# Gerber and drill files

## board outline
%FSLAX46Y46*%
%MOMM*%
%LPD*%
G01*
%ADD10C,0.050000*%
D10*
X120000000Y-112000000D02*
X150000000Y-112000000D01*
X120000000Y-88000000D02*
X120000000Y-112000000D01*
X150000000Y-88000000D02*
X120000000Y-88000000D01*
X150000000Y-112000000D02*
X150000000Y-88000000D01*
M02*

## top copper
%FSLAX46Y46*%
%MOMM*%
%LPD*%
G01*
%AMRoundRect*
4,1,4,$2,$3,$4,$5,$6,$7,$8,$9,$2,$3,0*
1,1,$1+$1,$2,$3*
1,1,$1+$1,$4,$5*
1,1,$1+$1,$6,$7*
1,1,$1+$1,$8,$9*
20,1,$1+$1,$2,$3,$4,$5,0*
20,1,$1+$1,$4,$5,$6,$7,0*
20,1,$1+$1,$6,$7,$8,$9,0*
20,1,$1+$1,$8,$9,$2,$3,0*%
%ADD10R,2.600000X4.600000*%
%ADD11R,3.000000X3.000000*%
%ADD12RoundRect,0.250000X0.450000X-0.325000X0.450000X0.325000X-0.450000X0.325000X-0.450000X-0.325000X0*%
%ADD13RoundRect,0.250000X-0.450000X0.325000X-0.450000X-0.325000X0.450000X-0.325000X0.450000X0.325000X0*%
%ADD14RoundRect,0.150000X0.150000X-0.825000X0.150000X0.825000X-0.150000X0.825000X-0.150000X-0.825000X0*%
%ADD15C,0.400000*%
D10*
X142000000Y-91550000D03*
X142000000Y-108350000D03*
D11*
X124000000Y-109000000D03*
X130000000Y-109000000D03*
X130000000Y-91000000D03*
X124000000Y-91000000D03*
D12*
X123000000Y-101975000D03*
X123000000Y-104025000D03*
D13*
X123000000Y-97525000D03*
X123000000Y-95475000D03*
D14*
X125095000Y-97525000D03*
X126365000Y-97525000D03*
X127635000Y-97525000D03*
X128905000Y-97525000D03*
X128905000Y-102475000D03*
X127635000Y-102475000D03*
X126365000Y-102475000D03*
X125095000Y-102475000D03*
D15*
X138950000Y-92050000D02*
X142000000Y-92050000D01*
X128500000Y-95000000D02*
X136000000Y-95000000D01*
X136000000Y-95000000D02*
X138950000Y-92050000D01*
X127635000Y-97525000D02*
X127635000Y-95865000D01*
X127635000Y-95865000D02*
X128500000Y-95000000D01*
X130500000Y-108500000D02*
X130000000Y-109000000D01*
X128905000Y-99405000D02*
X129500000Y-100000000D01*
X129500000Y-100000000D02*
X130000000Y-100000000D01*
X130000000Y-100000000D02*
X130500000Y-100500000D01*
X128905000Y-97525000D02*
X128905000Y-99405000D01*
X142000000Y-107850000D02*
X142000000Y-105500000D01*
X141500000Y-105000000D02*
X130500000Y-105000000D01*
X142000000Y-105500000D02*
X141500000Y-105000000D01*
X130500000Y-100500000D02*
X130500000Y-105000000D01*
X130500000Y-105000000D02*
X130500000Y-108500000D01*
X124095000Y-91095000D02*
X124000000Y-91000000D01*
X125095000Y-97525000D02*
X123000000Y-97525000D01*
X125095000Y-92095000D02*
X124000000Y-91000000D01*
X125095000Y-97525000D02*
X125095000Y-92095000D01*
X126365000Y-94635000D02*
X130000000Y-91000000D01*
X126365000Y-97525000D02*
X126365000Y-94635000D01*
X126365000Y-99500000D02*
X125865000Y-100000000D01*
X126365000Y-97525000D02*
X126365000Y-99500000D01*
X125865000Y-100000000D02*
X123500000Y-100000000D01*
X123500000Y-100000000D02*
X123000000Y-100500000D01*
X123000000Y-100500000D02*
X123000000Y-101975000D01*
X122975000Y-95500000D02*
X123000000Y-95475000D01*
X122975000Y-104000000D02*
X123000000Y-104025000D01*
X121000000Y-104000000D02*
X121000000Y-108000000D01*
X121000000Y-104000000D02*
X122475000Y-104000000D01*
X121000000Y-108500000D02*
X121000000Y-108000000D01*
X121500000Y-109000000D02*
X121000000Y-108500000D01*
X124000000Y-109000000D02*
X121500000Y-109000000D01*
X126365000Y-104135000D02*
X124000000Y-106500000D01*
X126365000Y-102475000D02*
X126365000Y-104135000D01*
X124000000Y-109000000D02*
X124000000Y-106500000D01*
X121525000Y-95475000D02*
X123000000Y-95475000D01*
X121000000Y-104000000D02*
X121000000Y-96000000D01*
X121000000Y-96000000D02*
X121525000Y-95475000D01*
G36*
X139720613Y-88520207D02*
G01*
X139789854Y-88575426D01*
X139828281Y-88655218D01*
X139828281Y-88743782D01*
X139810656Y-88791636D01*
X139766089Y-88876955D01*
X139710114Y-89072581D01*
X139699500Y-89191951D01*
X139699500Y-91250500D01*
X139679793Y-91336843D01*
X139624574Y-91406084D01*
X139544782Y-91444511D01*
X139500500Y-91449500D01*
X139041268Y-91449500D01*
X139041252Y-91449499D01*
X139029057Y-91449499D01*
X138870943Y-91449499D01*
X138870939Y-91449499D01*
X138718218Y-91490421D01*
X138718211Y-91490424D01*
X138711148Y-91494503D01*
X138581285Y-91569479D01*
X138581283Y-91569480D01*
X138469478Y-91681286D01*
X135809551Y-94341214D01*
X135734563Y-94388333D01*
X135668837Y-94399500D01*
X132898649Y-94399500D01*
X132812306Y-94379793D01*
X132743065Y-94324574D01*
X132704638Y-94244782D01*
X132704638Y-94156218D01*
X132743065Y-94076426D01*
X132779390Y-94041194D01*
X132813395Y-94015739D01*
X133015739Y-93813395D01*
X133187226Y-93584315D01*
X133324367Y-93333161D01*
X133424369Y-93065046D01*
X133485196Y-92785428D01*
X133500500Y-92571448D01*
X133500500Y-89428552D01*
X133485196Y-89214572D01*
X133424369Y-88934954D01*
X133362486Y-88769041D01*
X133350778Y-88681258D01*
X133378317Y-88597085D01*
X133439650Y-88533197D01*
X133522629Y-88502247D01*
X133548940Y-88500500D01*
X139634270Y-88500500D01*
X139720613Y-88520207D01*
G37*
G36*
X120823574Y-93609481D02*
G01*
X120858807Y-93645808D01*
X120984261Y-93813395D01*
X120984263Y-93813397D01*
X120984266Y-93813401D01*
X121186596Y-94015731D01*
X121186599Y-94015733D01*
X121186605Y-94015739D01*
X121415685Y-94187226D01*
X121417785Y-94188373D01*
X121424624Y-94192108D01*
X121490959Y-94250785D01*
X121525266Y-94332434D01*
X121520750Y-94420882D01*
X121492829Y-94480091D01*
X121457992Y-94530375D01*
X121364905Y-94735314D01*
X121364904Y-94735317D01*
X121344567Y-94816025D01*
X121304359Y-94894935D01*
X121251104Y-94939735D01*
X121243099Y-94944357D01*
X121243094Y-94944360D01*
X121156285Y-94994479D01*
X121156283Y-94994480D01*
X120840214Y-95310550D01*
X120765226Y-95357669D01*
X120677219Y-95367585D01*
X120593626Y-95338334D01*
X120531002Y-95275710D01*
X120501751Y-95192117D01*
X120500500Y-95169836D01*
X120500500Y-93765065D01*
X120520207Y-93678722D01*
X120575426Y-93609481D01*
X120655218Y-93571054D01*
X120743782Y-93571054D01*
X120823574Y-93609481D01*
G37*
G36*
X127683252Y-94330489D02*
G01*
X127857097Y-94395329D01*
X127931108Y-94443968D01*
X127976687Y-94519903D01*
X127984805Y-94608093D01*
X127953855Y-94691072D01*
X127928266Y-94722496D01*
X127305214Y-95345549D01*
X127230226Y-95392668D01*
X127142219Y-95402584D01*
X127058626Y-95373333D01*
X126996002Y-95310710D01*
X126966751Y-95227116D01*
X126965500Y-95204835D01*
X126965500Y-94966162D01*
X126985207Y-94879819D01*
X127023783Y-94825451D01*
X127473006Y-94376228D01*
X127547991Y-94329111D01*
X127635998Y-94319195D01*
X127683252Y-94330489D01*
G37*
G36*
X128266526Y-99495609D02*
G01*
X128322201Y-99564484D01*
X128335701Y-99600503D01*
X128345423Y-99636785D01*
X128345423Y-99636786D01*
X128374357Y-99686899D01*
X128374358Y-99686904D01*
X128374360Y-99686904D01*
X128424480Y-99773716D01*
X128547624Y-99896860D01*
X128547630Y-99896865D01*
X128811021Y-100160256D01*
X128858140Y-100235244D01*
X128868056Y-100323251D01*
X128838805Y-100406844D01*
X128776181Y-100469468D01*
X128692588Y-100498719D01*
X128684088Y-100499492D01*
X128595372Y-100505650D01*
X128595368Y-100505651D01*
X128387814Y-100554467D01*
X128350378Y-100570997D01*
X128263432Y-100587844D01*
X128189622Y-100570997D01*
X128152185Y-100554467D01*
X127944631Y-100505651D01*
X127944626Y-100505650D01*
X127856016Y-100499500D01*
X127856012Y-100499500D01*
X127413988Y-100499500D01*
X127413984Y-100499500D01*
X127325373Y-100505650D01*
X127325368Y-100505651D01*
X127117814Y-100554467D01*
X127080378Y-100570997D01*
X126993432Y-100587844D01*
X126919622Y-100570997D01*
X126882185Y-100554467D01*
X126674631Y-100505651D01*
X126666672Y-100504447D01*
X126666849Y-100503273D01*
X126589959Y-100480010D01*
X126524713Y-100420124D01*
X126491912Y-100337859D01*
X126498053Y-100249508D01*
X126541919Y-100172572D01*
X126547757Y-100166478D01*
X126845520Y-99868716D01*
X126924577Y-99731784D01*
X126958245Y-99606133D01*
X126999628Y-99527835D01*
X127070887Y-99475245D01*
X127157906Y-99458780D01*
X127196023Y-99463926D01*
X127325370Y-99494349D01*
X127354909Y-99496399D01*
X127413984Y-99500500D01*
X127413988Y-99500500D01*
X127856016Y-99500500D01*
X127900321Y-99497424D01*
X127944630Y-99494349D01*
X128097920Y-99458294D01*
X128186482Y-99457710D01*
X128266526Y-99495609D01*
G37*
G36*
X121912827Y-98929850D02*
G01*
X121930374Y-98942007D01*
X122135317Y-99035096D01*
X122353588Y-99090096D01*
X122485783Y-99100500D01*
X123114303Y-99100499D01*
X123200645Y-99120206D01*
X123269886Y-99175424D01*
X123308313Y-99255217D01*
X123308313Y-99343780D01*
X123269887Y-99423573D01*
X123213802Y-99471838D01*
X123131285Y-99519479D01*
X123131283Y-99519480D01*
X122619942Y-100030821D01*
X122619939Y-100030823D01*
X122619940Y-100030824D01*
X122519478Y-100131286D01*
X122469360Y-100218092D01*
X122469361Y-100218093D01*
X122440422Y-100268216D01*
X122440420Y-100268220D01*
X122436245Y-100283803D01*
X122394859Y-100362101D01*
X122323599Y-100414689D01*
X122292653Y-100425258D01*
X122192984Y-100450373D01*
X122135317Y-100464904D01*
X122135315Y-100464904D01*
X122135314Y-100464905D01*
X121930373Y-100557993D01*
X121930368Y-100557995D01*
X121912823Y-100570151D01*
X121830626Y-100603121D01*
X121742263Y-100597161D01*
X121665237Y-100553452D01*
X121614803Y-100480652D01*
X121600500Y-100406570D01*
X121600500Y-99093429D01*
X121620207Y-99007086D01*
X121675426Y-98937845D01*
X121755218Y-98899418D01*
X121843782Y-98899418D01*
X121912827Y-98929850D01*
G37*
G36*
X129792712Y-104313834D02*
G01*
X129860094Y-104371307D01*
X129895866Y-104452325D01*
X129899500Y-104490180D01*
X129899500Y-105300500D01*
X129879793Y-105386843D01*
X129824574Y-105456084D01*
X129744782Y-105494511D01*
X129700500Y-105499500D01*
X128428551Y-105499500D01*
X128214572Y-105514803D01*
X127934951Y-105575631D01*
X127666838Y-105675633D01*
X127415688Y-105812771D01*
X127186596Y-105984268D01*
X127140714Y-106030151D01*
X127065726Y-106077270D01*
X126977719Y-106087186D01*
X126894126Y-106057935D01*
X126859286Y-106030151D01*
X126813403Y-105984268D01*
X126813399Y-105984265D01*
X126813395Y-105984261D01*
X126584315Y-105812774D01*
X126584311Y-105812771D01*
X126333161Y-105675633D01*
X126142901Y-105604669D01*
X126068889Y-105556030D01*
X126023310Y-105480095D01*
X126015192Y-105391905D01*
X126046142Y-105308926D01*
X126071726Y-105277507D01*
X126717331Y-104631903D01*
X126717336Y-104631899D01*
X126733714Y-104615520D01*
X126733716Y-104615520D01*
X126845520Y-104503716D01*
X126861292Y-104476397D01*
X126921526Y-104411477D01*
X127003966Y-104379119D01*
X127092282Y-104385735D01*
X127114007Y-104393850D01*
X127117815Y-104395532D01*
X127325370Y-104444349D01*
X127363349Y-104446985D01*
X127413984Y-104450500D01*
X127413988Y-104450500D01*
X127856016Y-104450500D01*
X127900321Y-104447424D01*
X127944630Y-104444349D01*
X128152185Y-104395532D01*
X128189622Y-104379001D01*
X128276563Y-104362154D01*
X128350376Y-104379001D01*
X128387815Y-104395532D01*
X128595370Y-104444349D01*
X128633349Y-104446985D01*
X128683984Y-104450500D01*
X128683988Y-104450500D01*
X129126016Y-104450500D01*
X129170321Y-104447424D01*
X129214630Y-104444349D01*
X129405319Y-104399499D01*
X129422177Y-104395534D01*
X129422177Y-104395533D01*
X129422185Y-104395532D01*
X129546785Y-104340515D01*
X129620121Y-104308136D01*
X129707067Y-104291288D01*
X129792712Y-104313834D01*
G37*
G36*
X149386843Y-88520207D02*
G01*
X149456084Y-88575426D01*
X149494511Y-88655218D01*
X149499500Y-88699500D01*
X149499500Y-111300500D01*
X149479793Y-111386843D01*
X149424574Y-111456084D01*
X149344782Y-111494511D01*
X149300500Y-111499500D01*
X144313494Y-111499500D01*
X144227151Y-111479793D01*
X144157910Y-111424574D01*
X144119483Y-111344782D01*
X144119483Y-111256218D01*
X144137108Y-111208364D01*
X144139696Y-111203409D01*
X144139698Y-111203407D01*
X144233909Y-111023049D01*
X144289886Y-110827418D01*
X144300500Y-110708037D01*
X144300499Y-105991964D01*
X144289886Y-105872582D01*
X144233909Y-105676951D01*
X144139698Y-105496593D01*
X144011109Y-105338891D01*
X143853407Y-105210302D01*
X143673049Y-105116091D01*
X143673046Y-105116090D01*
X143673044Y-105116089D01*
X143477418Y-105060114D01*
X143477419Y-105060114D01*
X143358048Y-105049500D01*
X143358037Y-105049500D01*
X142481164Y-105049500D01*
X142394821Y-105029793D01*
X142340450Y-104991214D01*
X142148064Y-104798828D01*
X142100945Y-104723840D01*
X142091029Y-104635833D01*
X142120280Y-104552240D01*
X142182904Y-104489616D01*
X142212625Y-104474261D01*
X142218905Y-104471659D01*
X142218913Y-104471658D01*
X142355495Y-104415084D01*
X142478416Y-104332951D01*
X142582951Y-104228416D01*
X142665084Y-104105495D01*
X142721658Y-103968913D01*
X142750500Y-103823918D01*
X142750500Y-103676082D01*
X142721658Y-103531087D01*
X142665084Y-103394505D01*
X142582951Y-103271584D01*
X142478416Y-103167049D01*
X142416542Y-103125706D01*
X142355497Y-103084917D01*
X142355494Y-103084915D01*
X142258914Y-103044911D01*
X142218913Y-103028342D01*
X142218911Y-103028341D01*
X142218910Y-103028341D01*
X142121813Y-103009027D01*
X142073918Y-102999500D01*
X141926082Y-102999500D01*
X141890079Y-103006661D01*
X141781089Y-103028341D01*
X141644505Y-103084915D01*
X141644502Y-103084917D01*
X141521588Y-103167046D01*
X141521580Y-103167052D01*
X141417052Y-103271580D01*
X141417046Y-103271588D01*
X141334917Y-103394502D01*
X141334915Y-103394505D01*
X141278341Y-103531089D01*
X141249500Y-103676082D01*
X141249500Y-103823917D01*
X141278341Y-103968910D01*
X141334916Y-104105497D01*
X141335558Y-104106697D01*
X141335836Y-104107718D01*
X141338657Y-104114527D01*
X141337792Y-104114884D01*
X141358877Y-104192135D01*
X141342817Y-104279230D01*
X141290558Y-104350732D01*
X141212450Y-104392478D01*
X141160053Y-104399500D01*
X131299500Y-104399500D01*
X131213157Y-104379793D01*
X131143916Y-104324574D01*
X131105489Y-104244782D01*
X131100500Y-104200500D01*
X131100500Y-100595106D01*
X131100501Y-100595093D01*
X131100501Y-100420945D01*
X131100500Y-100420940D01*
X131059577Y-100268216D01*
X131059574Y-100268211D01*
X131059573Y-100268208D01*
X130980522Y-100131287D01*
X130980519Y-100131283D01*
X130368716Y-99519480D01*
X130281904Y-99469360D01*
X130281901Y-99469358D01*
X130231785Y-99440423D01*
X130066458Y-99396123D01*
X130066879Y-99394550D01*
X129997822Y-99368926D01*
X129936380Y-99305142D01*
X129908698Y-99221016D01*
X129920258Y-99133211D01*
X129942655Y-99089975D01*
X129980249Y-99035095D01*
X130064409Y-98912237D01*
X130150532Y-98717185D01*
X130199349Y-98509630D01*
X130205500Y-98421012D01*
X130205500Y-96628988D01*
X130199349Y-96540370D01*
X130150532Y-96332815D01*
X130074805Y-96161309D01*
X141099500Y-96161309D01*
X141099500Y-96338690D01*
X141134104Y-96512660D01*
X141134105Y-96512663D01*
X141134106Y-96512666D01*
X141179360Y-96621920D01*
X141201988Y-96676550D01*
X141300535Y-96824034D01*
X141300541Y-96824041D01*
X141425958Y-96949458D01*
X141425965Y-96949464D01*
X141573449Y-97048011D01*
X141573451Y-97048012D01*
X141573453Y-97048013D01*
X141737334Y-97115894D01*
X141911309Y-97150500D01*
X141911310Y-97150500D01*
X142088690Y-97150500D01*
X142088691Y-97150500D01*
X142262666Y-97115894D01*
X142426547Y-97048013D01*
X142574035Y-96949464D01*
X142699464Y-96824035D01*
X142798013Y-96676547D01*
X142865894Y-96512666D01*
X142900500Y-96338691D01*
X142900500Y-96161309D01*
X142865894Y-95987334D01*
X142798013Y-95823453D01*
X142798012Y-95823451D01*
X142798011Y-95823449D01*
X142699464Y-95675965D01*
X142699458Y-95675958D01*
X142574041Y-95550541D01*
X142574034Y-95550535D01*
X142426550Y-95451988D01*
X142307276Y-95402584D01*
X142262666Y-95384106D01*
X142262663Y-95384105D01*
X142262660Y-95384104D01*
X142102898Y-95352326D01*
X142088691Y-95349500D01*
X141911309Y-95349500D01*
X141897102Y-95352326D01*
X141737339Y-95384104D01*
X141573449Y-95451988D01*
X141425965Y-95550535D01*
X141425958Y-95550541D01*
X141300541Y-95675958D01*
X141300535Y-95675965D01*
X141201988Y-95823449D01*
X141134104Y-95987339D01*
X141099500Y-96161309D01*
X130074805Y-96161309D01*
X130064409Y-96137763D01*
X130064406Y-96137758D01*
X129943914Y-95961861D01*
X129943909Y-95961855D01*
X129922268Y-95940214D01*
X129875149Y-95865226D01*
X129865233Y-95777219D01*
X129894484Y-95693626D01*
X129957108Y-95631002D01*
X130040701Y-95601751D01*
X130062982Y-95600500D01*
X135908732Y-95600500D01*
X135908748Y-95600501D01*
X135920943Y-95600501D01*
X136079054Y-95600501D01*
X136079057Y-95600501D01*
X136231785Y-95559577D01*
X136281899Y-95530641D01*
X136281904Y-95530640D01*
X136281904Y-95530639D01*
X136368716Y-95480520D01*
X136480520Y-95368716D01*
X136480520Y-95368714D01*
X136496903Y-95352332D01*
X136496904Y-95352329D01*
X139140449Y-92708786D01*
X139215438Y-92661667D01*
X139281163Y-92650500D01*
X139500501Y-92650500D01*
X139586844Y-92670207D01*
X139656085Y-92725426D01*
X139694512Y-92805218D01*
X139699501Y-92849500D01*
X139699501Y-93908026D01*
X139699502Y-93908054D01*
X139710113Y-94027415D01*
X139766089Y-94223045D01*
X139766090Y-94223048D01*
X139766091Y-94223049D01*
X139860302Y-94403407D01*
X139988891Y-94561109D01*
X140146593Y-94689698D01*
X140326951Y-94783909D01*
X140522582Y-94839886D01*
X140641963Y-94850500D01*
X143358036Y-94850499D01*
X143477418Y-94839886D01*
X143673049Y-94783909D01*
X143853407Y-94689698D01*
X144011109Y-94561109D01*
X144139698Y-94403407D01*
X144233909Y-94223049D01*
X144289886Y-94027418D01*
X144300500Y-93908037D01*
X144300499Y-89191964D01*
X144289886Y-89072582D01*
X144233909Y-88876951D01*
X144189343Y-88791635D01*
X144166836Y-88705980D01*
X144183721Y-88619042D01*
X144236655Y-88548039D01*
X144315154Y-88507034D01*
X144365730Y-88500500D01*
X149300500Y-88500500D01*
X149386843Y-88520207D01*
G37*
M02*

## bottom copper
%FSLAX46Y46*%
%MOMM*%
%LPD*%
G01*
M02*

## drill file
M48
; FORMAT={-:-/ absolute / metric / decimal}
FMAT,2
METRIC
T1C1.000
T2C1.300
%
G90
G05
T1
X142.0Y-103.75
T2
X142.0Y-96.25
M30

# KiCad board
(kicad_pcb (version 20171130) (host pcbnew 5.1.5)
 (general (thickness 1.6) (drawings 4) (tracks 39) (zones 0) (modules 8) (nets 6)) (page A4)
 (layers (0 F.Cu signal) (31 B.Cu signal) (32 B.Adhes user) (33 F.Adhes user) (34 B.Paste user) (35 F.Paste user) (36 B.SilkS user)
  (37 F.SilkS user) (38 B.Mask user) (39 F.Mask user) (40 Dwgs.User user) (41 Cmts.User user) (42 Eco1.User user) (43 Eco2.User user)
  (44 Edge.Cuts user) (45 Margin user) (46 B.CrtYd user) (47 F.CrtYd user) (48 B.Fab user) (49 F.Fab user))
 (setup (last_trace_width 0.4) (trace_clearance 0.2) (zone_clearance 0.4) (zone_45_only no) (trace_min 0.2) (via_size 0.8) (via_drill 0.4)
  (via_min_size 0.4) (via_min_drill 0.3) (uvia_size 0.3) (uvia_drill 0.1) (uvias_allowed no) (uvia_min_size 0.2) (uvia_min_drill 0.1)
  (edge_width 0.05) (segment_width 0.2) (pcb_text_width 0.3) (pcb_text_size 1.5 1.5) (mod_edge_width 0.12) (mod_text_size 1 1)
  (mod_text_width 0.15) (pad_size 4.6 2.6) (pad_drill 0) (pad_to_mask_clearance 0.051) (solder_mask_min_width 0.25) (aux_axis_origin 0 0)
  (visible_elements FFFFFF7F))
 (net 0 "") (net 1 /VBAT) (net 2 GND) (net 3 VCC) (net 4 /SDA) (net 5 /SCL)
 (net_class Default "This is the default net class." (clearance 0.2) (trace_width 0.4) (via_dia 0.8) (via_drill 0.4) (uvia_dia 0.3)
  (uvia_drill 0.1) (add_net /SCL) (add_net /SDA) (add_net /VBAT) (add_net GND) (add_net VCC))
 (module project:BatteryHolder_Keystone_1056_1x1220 (layer F.Cu) (at 142 100.25 90)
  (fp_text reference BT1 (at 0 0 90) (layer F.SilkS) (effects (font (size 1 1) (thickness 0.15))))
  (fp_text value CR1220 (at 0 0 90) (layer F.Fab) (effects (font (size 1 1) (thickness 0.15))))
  (pad 1 smd rect (at 8.7 0 90) (size 4.6 2.6) (layers F.Cu F.Paste F.Mask) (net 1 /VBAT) (clearance 1))
  (pad 2 smd rect (at -8.1 0 90) (size 4.6 2.6) (layers F.Cu F.Paste F.Mask) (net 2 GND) (clearance 1))
  (pad "" np_thru_hole circle (at 4 0 90) (size 1.3 1.3) (drill 1.3) (layers *.Cu *.Mask))
  (pad "" np_thru_hole circle (at -3.5 0 90) (size 1 1) (drill 1) (layers *.Cu *.Mask)))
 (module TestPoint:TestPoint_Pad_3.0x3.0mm (layer F.Cu) (at 124 109 90) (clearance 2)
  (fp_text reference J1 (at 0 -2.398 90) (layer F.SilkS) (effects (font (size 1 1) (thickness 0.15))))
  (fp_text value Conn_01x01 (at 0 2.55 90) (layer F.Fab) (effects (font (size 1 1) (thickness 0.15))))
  (pad 1 smd rect (at 0 0 90) (size 3 3) (layers F.Cu F.Mask) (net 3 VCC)))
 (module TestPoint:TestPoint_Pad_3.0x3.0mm (layer F.Cu) (at 130 109 90)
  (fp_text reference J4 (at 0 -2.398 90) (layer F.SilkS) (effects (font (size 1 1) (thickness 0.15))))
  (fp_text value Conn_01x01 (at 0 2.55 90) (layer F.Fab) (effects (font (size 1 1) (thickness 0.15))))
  (pad 1 smd rect (at 0 0 90) (size 3 3) (layers F.Cu F.Mask) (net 2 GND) (clearance 2)))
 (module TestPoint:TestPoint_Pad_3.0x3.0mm (layer F.Cu) (at 130 91 90)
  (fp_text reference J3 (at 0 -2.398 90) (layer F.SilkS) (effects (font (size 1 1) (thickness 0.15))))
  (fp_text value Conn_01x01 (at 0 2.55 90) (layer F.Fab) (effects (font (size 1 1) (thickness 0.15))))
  (pad 1 smd rect (at 0 0 90) (size 3 3) (layers F.Cu F.Mask) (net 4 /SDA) (clearance 2)))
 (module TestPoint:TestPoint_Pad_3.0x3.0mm (layer F.Cu) (at 124 91 90) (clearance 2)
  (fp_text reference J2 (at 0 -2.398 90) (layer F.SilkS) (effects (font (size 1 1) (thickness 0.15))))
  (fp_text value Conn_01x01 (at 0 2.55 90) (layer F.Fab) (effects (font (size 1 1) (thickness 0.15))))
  (pad 1 smd rect (at 0 0 90) (size 3 3) (layers F.Cu F.Mask) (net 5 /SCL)))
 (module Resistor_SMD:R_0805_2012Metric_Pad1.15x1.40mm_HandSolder (layer F.Cu) (at 123 103 90) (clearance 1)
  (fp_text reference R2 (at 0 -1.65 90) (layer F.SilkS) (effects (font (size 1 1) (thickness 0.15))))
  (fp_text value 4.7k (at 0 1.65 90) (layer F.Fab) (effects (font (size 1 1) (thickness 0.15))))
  (pad 2 smd roundrect (at 1.025 0 90) (size 1.15 1.4) (layers F.Cu F.Paste F.Mask) (roundrect_rratio 0.217391) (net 4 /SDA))
  (pad 1 smd roundrect (at -1.025 0 90) (size 1.15 1.4) (layers F.Cu F.Paste F.Mask) (roundrect_rratio 0.217391) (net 3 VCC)))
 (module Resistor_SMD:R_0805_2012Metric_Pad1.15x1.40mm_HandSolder (layer F.Cu) (at 123 96.5 270) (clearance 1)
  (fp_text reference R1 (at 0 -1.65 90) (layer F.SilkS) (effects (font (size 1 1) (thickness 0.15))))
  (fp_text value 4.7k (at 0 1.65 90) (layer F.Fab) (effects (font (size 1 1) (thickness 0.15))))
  (pad 2 smd roundrect (at 1.025 0 270) (size 1.15 1.4) (layers F.Cu F.Paste F.Mask) (roundrect_rratio 0.217391) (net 5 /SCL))
  (pad 1 smd roundrect (at -1.025 0 270) (size 1.15 1.4) (layers F.Cu F.Paste F.Mask) (roundrect_rratio 0.217391) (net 3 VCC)))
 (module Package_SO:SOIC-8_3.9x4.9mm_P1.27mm (layer F.Cu) (at 127 100 90) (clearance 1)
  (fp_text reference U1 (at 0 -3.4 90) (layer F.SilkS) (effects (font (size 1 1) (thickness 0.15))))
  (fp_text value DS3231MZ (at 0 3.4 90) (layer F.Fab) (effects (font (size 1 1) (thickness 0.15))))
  (pad 8 smd roundrect (at 2.475 -1.905 90) (size 1.95 0.6) (layers F.Cu F.Paste F.Mask) (roundrect_rratio 0.25) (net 5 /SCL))
  (pad 7 smd roundrect (at 2.475 -0.635 90) (size 1.95 0.6) (layers F.Cu F.Paste F.Mask) (roundrect_rratio 0.25) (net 4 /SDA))
  (pad 6 smd roundrect (at 2.475 0.635 90) (size 1.95 0.6) (layers F.Cu F.Paste F.Mask) (roundrect_rratio 0.25) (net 1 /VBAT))
  (pad 5 smd roundrect (at 2.475 1.905 90) (size 1.95 0.6) (layers F.Cu F.Paste F.Mask) (roundrect_rratio 0.25) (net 2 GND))
  (pad 4 smd roundrect (at -2.475 1.905 90) (size 1.95 0.6) (layers F.Cu F.Paste F.Mask) (roundrect_rratio 0.25))
  (pad 3 smd roundrect (at -2.475 0.635 90) (size 1.95 0.6) (layers F.Cu F.Paste F.Mask) (roundrect_rratio 0.25))
  (pad 2 smd roundrect (at -2.475 -0.635 90) (size 1.95 0.6) (layers F.Cu F.Paste F.Mask) (roundrect_rratio 0.25) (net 3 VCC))
  (pad 1 smd roundrect (at -2.475 -1.905 90) (size 1.95 0.6) (layers F.Cu F.Paste F.Mask) (roundrect_rratio 0.25)))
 (gr_line (start 120 112) (end 150 112) (layer Edge.Cuts) (width 0.05))
 (gr_line (start 120 88) (end 120 112) (layer Edge.Cuts) (width 0.05))
 (gr_line (start 150 88) (end 120 88) (layer Edge.Cuts) (width 0.05))
 (gr_line (start 150 112) (end 150 88) (layer Edge.Cuts) (width 0.05))
 (segment (start 138.95 92.05) (end 142 92.05) (width 0.4) (layer F.Cu) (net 1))
 (segment (start 128.5 95) (end 136 95) (width 0.4) (layer F.Cu) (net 1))
 (segment (start 136 95) (end 138.95 92.05) (width 0.4) (layer F.Cu) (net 1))
 (segment (start 127.635 97.525) (end 127.635 95.865) (width 0.4) (layer F.Cu) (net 1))
 (segment (start 127.635 95.865) (end 128.5 95) (width 0.4) (layer F.Cu) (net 1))
 (segment (start 130.5 108.5) (end 130 109) (width 0.4) (layer F.Cu) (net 2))
 (segment (start 128.905 99.405) (end 129.5 100) (width 0.4) (layer F.Cu) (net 2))
 (segment (start 129.5 100) (end 130 100) (width 0.4) (layer F.Cu) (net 2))
 (segment (start 130 100) (end 130.5 100.5) (width 0.4) (layer F.Cu) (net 2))
 (segment (start 128.905 97.525) (end 128.905 99.405) (width 0.4) (layer F.Cu) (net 2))
 (segment (start 142 107.85) (end 142 105.5) (width 0.4) (layer F.Cu) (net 2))
 (segment (start 141.5 105) (end 130.5 105) (width 0.4) (layer F.Cu) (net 2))
 (segment (start 142 105.5) (end 141.5 105) (width 0.4) (layer F.Cu) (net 2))
 (segment (start 130.5 100.5) (end 130.5 105) (width 0.4) (layer F.Cu) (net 2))
 (segment (start 130.5 105) (end 130.5 108.5) (width 0.4) (layer F.Cu) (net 2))
 (segment (start 124.095 91.095) (end 124 91) (width 0.4) (layer F.Cu) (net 5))
 (segment (start 125.095 97.525) (end 123 97.525) (width 0.4) (layer F.Cu) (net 5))
 (segment (start 125.095 92.095) (end 124 91) (width 0.4) (layer F.Cu) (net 5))
 (segment (start 125.095 97.525) (end 125.095 92.095) (width 0.4) (layer F.Cu) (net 5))
 (segment (start 126.365 94.635) (end 130 91) (width 0.4) (layer F.Cu) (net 4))
 (segment (start 126.365 97.525) (end 126.365 94.635) (width 0.4) (layer F.Cu) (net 4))
 (segment (start 126.365 99.5) (end 125.865 100) (width 0.4) (layer F.Cu) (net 4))
 (segment (start 126.365 97.525) (end 126.365 99.5) (width 0.4) (layer F.Cu) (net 4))
 (segment (start 125.865 100) (end 123.5 100) (width 0.4) (layer F.Cu) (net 4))
 (segment (start 123.5 100) (end 123 100.5) (width 0.4) (layer F.Cu) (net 4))
 (segment (start 123 100.5) (end 123 101.975) (width 0.4) (layer F.Cu) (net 4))
 (segment (start 122.975 95.5) (end 123 95.475) (width 0.4) (layer F.Cu) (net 3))
 (segment (start 122.975 104) (end 123 104.025) (width 0.4) (layer F.Cu) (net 3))
 (segment (start 121 104) (end 121 108) (width 0.4) (layer F.Cu) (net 3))
 (segment (start 121 104) (end 122.475 104) (width 0.4) (layer F.Cu) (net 3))
 (segment (start 121 108.5) (end 121 108) (width 0.4) (layer F.Cu) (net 3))
 (segment (start 121.5 109) (end 121 108.5) (width 0.4) (layer F.Cu) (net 3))
 (segment (start 124 109) (end 121.5 109) (width 0.4) (layer F.Cu) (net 3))
 (segment (start 126.365 104.135) (end 124 106.5) (width 0.4) (layer F.Cu) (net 3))
 (segment (start 126.365 102.475) (end 126.365 104.135) (width 0.4) (layer F.Cu) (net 3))
 (segment (start 124 109) (end 124 106.5) (width 0.4) (layer F.Cu) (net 3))
 (segment (start 121.525 95.475) (end 123 95.475) (width 0.4) (layer F.Cu) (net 3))
 (segment (start 121 104) (end 121 96) (width 0.4) (layer F.Cu) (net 3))
 (segment (start 121 96) (end 121.525 95.475) (width 0.4) (layer F.Cu) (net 3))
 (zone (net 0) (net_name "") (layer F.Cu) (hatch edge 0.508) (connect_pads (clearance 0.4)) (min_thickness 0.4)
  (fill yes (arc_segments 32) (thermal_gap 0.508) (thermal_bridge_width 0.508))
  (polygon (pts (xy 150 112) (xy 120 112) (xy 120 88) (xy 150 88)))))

